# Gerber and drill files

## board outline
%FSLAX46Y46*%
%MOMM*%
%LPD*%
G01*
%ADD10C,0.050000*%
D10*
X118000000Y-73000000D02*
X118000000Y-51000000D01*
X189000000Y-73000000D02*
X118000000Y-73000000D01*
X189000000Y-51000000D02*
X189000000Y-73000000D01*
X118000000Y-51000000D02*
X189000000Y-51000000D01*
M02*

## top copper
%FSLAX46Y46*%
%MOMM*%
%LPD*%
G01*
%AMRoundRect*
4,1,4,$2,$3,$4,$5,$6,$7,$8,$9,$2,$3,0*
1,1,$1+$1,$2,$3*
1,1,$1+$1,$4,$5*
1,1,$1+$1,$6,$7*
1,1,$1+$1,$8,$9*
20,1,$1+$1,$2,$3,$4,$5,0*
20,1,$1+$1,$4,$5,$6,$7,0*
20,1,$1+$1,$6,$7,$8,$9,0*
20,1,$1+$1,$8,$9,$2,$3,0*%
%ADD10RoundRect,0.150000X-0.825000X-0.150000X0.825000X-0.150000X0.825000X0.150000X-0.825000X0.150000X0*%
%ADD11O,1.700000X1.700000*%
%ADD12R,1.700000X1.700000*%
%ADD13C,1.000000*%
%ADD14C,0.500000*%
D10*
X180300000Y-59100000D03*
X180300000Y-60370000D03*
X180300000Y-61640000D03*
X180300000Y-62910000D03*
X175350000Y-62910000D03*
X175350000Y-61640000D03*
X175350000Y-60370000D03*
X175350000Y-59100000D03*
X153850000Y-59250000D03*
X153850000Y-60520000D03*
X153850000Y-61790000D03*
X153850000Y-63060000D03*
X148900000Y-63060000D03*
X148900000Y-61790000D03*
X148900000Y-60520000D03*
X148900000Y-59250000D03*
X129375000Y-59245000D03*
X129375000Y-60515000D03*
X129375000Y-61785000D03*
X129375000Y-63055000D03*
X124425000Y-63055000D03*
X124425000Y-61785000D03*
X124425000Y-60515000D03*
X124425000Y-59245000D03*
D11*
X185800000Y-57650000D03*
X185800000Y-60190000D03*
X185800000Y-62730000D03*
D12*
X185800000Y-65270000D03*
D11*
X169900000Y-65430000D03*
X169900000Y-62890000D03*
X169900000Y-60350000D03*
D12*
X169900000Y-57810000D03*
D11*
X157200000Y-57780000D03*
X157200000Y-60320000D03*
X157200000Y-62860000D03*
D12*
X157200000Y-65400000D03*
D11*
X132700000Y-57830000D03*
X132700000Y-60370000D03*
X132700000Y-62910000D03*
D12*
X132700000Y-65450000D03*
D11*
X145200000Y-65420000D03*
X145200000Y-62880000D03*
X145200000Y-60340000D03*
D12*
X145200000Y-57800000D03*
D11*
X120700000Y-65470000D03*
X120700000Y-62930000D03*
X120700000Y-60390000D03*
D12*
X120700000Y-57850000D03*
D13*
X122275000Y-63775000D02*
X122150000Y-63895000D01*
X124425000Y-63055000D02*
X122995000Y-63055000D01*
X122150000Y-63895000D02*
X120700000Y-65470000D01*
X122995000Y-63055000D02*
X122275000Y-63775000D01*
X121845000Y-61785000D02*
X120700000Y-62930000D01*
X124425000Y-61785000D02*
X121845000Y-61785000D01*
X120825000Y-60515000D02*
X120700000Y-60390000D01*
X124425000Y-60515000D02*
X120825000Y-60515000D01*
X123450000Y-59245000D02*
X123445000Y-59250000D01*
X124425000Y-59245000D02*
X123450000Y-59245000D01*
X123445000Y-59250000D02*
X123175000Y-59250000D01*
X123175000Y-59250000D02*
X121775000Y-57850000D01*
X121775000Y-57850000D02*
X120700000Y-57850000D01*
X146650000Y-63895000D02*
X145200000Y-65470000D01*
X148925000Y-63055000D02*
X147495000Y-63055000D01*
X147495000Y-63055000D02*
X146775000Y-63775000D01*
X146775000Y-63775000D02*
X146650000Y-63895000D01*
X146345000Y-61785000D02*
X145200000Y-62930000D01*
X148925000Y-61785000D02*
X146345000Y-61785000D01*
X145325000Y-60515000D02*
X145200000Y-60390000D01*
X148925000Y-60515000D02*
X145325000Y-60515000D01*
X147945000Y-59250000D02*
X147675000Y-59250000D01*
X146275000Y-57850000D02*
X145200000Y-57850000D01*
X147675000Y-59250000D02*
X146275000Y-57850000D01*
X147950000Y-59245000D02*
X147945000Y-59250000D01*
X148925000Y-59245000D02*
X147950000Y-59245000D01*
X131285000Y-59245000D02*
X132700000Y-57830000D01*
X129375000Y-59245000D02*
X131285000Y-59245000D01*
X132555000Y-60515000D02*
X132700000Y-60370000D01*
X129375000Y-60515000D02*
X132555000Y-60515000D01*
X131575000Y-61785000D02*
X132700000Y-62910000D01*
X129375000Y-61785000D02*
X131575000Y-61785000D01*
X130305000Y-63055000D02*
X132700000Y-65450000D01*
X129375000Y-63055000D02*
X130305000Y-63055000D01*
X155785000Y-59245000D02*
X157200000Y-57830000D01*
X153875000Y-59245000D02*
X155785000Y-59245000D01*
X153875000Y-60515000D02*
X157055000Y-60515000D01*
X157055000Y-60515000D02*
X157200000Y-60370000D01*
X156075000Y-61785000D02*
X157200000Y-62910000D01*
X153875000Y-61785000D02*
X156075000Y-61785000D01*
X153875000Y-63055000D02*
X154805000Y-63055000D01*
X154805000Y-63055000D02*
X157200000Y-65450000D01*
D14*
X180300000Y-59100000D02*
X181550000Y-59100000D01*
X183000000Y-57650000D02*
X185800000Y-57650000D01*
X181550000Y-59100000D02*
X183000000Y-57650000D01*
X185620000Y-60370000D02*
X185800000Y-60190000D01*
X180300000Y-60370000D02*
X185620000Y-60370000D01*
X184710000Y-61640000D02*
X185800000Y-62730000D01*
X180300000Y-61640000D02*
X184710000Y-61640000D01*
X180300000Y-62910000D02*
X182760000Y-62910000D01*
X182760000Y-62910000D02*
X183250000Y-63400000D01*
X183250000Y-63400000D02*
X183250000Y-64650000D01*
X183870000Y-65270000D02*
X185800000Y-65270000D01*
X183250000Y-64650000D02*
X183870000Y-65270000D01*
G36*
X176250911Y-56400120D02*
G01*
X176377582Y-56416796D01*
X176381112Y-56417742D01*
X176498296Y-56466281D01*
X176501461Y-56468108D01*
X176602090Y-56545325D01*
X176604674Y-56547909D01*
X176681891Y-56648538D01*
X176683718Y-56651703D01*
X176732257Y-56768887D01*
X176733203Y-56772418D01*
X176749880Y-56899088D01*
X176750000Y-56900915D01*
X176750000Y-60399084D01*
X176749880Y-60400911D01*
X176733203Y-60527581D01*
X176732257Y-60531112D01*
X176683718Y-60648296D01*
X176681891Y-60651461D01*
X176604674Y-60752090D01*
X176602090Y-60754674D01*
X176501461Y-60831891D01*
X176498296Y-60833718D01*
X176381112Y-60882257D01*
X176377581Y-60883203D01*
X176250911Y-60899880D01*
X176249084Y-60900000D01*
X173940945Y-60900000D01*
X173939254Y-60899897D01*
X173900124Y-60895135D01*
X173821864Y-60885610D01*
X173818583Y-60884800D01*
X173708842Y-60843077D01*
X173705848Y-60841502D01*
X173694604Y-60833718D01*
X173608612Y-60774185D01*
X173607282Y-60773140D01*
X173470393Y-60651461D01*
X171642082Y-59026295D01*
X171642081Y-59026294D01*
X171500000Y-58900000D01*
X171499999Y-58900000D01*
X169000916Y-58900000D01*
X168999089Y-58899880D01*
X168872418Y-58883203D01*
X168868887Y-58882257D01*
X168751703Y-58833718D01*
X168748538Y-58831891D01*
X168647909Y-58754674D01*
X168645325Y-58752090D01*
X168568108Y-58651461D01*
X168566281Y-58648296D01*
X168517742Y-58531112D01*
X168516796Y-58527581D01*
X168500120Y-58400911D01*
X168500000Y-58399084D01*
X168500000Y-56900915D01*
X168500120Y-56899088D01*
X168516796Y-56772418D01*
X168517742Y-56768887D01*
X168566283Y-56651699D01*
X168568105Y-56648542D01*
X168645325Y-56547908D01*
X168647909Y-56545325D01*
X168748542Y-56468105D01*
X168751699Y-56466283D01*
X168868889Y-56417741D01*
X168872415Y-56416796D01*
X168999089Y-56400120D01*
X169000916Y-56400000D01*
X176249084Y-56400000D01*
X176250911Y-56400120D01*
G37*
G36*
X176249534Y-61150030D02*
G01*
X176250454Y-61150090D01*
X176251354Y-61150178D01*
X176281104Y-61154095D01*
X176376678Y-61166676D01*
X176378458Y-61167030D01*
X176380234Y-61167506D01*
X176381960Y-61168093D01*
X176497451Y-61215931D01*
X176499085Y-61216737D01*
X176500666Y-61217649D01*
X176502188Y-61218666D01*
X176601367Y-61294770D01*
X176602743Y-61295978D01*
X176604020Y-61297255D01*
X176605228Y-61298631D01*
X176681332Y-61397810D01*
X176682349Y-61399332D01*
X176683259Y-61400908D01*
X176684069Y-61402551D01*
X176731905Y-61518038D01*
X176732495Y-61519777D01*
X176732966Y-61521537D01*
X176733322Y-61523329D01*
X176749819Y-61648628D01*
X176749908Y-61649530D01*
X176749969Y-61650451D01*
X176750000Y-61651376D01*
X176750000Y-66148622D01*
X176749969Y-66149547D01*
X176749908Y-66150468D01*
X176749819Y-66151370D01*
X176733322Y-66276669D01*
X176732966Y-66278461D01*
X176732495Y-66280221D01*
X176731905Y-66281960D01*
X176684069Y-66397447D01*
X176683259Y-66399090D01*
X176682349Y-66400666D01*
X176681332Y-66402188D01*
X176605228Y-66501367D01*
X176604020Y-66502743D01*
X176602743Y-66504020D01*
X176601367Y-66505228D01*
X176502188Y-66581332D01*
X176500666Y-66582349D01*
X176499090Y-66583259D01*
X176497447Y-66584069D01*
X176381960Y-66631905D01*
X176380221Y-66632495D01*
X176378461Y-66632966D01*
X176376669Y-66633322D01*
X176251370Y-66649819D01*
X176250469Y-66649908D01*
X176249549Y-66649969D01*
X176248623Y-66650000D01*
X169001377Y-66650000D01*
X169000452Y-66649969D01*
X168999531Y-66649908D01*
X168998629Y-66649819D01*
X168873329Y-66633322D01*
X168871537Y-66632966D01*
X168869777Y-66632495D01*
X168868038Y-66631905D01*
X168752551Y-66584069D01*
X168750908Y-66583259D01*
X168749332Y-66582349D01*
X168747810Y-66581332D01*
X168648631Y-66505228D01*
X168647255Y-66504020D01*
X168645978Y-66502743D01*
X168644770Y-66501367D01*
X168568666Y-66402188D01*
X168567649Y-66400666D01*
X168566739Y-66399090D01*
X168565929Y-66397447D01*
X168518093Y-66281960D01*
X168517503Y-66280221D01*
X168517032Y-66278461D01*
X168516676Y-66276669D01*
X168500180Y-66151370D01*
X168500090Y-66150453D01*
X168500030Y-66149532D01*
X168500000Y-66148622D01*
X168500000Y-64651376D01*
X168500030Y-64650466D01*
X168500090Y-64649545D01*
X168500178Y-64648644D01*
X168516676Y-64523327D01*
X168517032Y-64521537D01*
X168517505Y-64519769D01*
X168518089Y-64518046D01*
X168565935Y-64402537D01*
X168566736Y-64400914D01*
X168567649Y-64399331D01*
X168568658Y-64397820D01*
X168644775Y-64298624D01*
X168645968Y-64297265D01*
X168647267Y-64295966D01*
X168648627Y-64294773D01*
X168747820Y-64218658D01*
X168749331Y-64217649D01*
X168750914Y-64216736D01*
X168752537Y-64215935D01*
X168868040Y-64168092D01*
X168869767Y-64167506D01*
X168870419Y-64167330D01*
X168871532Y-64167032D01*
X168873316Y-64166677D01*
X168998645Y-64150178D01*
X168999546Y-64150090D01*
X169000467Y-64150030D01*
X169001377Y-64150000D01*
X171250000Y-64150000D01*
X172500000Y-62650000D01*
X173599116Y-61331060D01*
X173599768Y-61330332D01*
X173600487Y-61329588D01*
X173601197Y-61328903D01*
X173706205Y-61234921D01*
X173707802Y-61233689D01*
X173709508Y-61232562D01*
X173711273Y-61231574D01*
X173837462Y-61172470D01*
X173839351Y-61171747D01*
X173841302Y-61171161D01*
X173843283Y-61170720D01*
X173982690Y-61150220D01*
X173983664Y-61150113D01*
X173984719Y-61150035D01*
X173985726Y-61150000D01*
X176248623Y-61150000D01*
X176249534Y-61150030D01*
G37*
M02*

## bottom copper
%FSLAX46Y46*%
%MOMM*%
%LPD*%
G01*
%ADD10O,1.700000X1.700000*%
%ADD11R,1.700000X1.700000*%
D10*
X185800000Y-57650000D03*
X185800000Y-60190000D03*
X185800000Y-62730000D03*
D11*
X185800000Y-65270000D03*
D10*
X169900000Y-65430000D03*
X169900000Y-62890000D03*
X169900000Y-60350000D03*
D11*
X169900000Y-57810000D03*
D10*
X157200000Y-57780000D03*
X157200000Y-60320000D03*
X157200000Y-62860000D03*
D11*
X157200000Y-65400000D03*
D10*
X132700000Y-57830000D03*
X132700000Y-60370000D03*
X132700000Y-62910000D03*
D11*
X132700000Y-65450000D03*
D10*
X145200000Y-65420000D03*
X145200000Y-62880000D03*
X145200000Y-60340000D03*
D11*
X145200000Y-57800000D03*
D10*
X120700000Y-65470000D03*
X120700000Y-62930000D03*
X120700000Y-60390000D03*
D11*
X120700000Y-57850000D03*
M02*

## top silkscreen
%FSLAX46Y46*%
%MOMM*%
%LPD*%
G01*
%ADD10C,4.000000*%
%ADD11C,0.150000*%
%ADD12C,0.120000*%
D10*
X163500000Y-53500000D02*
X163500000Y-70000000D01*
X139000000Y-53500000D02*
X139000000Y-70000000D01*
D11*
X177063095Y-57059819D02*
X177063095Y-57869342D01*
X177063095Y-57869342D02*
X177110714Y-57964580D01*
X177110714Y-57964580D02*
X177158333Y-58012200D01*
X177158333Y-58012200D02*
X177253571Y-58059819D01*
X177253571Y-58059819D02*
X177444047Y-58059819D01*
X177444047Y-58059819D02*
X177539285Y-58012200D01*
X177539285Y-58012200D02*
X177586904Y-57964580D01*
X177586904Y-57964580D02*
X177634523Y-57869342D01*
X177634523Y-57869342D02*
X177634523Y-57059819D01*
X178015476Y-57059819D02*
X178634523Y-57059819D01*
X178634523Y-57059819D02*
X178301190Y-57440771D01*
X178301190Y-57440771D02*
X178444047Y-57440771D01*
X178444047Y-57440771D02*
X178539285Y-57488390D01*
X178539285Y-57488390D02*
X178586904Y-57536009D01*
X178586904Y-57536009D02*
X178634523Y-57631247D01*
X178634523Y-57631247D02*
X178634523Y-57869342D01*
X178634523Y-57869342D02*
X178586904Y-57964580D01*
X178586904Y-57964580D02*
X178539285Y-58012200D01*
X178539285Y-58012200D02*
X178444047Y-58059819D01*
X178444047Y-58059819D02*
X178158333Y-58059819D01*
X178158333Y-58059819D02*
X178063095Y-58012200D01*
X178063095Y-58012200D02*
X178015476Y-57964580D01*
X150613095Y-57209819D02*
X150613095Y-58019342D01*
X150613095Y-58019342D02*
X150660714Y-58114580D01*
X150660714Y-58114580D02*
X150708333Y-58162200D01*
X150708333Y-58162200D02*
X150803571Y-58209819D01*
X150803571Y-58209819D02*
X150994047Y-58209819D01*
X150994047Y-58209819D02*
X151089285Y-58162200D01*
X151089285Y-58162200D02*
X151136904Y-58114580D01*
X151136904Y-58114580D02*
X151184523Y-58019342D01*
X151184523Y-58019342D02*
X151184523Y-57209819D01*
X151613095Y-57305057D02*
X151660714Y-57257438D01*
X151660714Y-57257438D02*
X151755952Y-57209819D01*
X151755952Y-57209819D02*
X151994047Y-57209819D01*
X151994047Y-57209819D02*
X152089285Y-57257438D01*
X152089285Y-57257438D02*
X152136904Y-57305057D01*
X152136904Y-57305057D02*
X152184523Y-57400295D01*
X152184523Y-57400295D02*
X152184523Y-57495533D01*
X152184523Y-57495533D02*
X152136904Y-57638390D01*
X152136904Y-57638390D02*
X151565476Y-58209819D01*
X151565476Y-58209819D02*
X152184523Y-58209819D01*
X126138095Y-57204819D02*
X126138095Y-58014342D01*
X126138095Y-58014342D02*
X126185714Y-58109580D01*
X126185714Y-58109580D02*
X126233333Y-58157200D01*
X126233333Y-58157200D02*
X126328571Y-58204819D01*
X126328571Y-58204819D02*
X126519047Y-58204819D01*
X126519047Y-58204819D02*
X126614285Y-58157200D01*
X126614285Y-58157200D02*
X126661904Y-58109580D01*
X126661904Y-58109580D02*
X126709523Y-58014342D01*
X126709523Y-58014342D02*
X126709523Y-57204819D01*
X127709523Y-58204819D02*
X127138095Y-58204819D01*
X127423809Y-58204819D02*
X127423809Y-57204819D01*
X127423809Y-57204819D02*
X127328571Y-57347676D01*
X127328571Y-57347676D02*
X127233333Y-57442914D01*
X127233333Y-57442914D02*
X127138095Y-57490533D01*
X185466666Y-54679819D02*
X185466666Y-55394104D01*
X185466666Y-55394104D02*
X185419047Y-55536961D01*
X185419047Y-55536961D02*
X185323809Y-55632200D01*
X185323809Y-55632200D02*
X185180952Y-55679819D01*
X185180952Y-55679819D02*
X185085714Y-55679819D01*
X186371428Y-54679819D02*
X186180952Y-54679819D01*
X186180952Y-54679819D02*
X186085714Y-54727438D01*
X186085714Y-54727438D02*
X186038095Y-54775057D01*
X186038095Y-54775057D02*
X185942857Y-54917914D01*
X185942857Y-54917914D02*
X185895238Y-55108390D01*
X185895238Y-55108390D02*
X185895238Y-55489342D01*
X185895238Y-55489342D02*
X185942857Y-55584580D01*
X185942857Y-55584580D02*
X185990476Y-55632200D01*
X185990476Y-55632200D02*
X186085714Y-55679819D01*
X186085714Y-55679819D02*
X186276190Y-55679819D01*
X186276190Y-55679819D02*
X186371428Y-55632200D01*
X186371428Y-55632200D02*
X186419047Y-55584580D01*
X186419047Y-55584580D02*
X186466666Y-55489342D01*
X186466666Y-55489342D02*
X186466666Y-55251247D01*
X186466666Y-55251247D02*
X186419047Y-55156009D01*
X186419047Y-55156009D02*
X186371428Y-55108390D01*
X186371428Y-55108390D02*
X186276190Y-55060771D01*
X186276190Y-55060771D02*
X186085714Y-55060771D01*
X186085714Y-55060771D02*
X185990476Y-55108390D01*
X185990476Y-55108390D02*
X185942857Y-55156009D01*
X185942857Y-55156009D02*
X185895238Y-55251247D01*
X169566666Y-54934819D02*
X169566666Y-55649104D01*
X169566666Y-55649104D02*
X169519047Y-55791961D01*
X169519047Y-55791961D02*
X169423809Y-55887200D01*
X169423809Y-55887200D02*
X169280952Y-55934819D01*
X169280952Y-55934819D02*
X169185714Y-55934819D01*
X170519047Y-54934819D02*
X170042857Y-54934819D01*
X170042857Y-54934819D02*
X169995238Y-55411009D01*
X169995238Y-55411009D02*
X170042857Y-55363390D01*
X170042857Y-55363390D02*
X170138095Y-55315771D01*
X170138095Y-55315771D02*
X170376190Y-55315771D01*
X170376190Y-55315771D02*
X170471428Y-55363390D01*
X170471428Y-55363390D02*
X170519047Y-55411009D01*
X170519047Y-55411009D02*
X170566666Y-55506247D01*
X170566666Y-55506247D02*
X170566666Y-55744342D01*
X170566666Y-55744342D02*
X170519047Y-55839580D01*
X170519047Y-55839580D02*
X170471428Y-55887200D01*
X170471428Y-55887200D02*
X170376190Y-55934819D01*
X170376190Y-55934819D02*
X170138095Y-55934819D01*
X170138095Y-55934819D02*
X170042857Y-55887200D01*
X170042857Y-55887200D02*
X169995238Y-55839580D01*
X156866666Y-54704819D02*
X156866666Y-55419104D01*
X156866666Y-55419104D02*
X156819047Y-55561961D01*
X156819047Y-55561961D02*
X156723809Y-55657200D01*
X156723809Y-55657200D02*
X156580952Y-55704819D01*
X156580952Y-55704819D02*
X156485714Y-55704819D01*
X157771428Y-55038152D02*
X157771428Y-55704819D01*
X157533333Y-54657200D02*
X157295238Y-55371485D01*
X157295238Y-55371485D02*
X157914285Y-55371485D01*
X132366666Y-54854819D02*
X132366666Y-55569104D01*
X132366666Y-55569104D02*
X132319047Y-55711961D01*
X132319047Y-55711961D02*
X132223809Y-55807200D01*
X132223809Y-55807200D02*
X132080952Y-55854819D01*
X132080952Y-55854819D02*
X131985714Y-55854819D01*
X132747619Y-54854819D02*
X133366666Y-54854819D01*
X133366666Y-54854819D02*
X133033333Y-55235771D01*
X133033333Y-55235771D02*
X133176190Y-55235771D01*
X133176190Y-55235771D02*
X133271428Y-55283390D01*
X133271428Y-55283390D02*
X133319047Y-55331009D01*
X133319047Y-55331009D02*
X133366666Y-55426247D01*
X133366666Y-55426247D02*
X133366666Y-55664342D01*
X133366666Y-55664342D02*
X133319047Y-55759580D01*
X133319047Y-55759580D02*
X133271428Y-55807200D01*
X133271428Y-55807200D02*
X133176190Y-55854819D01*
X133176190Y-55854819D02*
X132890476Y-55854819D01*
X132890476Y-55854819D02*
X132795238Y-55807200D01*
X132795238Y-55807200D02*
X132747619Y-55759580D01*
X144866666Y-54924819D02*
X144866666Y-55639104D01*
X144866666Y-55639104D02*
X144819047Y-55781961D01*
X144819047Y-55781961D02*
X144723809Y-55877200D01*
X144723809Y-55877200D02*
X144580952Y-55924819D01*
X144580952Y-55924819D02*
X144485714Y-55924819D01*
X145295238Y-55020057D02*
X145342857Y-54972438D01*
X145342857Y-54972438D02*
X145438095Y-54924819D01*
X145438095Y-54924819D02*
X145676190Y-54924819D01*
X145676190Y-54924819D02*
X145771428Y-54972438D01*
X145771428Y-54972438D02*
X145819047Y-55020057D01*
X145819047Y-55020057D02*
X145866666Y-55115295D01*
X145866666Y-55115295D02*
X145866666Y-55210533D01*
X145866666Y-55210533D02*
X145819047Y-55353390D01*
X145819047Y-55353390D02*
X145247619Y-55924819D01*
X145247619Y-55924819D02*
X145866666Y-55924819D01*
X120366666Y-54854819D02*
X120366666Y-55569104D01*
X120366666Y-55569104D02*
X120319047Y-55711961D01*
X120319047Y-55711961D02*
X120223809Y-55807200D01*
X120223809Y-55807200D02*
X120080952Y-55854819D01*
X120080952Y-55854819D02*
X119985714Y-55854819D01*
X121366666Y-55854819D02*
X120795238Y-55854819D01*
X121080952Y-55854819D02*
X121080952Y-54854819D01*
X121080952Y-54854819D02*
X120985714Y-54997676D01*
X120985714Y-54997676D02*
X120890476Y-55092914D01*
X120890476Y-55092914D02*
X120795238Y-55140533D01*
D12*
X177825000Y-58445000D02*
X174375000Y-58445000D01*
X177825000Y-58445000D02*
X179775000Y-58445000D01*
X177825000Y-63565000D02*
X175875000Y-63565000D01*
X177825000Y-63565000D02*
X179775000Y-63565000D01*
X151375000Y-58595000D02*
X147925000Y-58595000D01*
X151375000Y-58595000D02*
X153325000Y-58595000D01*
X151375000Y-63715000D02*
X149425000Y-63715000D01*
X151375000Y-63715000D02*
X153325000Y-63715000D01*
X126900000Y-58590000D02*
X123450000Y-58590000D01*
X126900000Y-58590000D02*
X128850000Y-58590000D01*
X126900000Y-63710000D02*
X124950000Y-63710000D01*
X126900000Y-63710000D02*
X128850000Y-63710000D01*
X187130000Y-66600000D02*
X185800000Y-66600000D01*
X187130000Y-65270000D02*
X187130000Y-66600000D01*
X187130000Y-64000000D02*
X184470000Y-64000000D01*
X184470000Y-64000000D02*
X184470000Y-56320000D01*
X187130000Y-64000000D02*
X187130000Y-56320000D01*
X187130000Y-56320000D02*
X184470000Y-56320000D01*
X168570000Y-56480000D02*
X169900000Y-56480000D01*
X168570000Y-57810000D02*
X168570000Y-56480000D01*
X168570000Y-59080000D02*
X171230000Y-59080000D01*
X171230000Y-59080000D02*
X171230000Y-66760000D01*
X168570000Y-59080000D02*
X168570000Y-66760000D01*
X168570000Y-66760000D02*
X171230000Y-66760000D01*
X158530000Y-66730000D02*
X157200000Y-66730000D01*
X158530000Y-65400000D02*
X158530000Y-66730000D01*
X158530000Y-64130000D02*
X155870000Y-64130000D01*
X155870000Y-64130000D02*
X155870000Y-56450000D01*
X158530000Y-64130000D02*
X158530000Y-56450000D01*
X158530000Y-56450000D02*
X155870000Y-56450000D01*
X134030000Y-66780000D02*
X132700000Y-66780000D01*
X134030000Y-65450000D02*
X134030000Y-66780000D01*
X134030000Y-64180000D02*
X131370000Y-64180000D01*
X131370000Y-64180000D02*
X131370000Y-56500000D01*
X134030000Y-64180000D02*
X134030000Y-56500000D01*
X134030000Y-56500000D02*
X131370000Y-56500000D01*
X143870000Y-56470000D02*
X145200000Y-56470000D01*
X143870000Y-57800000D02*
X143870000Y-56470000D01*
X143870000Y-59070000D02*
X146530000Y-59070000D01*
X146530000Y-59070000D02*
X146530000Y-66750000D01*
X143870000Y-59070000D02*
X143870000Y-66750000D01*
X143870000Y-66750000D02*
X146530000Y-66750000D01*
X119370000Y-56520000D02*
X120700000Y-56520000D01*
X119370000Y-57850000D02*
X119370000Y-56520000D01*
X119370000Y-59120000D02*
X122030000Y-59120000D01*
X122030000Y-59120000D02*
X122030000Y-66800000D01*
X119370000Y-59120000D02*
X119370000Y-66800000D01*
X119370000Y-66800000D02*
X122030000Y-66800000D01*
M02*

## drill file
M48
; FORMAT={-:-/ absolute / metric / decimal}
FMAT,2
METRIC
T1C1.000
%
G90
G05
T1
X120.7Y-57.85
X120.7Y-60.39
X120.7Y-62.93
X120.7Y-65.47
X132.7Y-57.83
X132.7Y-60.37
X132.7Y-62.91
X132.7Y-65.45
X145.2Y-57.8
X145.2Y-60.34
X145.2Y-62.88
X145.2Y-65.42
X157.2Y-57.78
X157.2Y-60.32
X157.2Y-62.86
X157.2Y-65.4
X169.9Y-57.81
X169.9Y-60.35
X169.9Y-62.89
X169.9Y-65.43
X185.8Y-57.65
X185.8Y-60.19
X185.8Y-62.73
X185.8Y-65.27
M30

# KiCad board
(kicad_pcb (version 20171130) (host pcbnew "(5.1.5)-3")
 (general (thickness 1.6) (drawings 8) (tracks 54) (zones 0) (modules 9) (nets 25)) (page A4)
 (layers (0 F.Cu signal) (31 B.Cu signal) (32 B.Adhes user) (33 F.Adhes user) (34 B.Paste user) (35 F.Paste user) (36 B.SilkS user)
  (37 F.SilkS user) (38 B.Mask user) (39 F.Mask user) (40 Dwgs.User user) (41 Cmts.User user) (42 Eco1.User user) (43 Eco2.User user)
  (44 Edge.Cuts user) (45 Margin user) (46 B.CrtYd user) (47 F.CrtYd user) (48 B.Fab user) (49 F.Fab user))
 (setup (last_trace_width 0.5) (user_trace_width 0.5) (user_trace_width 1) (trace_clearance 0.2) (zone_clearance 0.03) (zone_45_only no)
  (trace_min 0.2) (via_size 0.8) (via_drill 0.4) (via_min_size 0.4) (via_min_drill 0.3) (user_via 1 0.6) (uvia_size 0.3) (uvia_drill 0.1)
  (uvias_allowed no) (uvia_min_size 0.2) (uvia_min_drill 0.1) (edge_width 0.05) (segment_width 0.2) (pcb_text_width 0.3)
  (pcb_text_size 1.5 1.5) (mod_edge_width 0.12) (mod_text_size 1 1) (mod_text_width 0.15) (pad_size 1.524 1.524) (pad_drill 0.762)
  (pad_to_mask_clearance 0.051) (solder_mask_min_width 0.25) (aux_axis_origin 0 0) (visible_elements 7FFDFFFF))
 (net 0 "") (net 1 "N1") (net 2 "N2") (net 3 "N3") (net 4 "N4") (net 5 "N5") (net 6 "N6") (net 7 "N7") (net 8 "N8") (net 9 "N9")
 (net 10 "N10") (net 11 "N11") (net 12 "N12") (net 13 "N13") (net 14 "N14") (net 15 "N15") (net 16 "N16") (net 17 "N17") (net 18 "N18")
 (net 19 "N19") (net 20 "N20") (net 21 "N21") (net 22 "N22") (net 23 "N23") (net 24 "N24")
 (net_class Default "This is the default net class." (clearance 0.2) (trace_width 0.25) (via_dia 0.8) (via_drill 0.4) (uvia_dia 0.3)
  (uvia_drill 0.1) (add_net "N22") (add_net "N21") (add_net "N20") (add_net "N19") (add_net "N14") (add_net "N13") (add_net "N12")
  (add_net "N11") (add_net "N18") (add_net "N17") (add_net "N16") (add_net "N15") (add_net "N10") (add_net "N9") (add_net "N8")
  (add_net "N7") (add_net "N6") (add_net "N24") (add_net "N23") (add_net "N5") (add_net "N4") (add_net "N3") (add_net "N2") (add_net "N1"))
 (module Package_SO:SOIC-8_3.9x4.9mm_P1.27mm (layer F.Cu) (at 177.825 61.005)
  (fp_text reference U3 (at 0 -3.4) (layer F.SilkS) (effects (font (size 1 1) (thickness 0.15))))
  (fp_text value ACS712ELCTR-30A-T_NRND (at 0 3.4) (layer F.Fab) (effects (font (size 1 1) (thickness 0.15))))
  (fp_line (start 0 -2.56) (end -3.45 -2.56) (layer F.SilkS) (width 0.12))
  (fp_line (start 0 -2.56) (end 1.95 -2.56) (layer F.SilkS) (width 0.12))
  (fp_line (start 0 2.56) (end -1.95 2.56) (layer F.SilkS) (width 0.12))
  (fp_line (start 0 2.56) (end 1.95 2.56) (layer F.SilkS) (width 0.12))
  (pad 8 smd roundrect (at 2.475 -1.905) (size 1.95 0.6) (layers F.Cu F.Paste F.Mask) (roundrect_rratio 0.25) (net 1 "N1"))
  (pad 7 smd roundrect (at 2.475 -0.635) (size 1.95 0.6) (layers F.Cu F.Paste F.Mask) (roundrect_rratio 0.25) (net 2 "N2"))
  (pad 6 smd roundrect (at 2.475 0.635) (size 1.95 0.6) (layers F.Cu F.Paste F.Mask) (roundrect_rratio 0.25) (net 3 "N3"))
  (pad 5 smd roundrect (at 2.475 1.905) (size 1.95 0.6) (layers F.Cu F.Paste F.Mask) (roundrect_rratio 0.25) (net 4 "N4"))
  (pad 4 smd roundrect (at -2.475 1.905) (size 1.95 0.6) (layers F.Cu F.Paste F.Mask) (roundrect_rratio 0.25) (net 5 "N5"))
  (pad 3 smd roundrect (at -2.475 0.635) (size 1.95 0.6) (layers F.Cu F.Paste F.Mask) (roundrect_rratio 0.25) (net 5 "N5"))
  (pad 2 smd roundrect (at -2.475 -0.635) (size 1.95 0.6) (layers F.Cu F.Paste F.Mask) (roundrect_rratio 0.25) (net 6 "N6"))
  (pad 1 smd roundrect (at -2.475 -1.905) (size 1.95 0.6) (layers F.Cu F.Paste F.Mask) (roundrect_rratio 0.25) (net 6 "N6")))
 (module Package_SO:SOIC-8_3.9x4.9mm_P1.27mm (layer F.Cu) (at 151.375 61.155)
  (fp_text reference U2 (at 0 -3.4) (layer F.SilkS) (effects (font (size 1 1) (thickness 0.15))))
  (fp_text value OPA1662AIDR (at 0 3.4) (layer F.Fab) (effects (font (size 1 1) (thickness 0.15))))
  (fp_line (start 0 -2.56) (end -3.45 -2.56) (layer F.SilkS) (width 0.12))
  (fp_line (start 0 -2.56) (end 1.95 -2.56) (layer F.SilkS) (width 0.12))
  (fp_line (start 0 2.56) (end -1.95 2.56) (layer F.SilkS) (width 0.12))
  (fp_line (start 0 2.56) (end 1.95 2.56) (layer F.SilkS) (width 0.12))
  (pad 8 smd roundrect (at 2.475 -1.905) (size 1.95 0.6) (layers F.Cu F.Paste F.Mask) (roundrect_rratio 0.25) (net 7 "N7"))
  (pad 7 smd roundrect (at 2.475 -0.635) (size 1.95 0.6) (layers F.Cu F.Paste F.Mask) (roundrect_rratio 0.25) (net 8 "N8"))
  (pad 6 smd roundrect (at 2.475 0.635) (size 1.95 0.6) (layers F.Cu F.Paste F.Mask) (roundrect_rratio 0.25) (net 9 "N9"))
  (pad 5 smd roundrect (at 2.475 1.905) (size 1.95 0.6) (layers F.Cu F.Paste F.Mask) (roundrect_rratio 0.25) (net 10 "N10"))
  (pad 4 smd roundrect (at -2.475 1.905) (size 1.95 0.6) (layers F.Cu F.Paste F.Mask) (roundrect_rratio 0.25) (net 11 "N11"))
  (pad 3 smd roundrect (at -2.475 0.635) (size 1.95 0.6) (layers F.Cu F.Paste F.Mask) (roundrect_rratio 0.25) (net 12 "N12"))
  (pad 2 smd roundrect (at -2.475 -0.635) (size 1.95 0.6) (layers F.Cu F.Paste F.Mask) (roundrect_rratio 0.25) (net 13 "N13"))
  (pad 1 smd roundrect (at -2.475 -1.905) (size 1.95 0.6) (layers F.Cu F.Paste F.Mask) (roundrect_rratio 0.25) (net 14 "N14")))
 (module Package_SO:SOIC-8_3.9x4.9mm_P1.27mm (layer F.Cu) (at 126.9 61.15)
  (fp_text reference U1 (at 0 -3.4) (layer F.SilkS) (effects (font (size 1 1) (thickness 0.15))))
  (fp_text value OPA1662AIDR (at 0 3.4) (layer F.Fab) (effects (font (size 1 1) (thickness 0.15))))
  (fp_line (start 0 -2.56) (end -3.45 -2.56) (layer F.SilkS) (width 0.12))
  (fp_line (start 0 -2.56) (end 1.95 -2.56) (layer F.SilkS) (width 0.12))
  (fp_line (start 0 2.56) (end -1.95 2.56) (layer F.SilkS) (width 0.12))
  (fp_line (start 0 2.56) (end 1.95 2.56) (layer F.SilkS) (width 0.12))
  (pad 8 smd roundrect (at 2.475 -1.905) (size 1.95 0.6) (layers F.Cu F.Paste F.Mask) (roundrect_rratio 0.25) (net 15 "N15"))
  (pad 7 smd roundrect (at 2.475 -0.635) (size 1.95 0.6) (layers F.Cu F.Paste F.Mask) (roundrect_rratio 0.25) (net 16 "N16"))
  (pad 6 smd roundrect (at 2.475 0.635) (size 1.95 0.6) (layers F.Cu F.Paste F.Mask) (roundrect_rratio 0.25) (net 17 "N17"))
  (pad 5 smd roundrect (at 2.475 1.905) (size 1.95 0.6) (layers F.Cu F.Paste F.Mask) (roundrect_rratio 0.25) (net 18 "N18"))
  (pad 4 smd roundrect (at -2.475 1.905) (size 1.95 0.6) (layers F.Cu F.Paste F.Mask) (roundrect_rratio 0.25) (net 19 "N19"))
  (pad 3 smd roundrect (at -2.475 0.635) (size 1.95 0.6) (layers F.Cu F.Paste F.Mask) (roundrect_rratio 0.25) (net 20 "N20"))
  (pad 2 smd roundrect (at -2.475 -0.635) (size 1.95 0.6) (layers F.Cu F.Paste F.Mask) (roundrect_rratio 0.25) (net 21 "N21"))
  (pad 1 smd roundrect (at -2.475 -1.905) (size 1.95 0.6) (layers F.Cu F.Paste F.Mask) (roundrect_rratio 0.25) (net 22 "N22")))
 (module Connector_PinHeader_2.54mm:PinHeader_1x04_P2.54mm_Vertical (layer F.Cu) (at 185.8 65.27 180)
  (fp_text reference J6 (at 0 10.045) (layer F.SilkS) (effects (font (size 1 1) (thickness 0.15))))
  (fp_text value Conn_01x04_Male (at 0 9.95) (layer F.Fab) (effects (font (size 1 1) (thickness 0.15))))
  (fp_line (start -1.33 -1.33) (end 0 -1.33) (layer F.SilkS) (width 0.12))
  (fp_line (start -1.33 0) (end -1.33 -1.33) (layer F.SilkS) (width 0.12))
  (fp_line (start -1.33 1.27) (end 1.33 1.27) (layer F.SilkS) (width 0.12))
  (fp_line (start 1.33 1.27) (end 1.33 8.95) (layer F.SilkS) (width 0.12))
  (fp_line (start -1.33 1.27) (end -1.33 8.95) (layer F.SilkS) (width 0.12))
  (fp_line (start -1.33 8.95) (end 1.33 8.95) (layer F.SilkS) (width 0.12))
  (pad 4 thru_hole oval (at 0 7.62 180) (size 1.7 1.7) (drill 1) (layers *.Cu *.Mask) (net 1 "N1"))
  (pad 3 thru_hole oval (at 0 5.08 180) (size 1.7 1.7) (drill 1) (layers *.Cu *.Mask) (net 2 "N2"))
  (pad 2 thru_hole oval (at 0 2.54 180) (size 1.7 1.7) (drill 1) (layers *.Cu *.Mask) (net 3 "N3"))
  (pad 1 thru_hole rect (at 0 0 180) (size 1.7 1.7) (drill 1) (layers *.Cu *.Mask) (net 4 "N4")))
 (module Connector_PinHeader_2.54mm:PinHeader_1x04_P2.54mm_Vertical (layer F.Cu) (at 169.9 57.81)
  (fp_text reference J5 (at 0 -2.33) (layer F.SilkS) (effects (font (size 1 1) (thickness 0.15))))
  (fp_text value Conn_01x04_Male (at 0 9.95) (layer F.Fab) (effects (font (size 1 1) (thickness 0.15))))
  (fp_line (start -1.33 -1.33) (end 0 -1.33) (layer F.SilkS) (width 0.12))
  (fp_line (start -1.33 0) (end -1.33 -1.33) (layer F.SilkS) (width 0.12))
  (fp_line (start -1.33 1.27) (end 1.33 1.27) (layer F.SilkS) (width 0.12))
  (fp_line (start 1.33 1.27) (end 1.33 8.95) (layer F.SilkS) (width 0.12))
  (fp_line (start -1.33 1.27) (end -1.33 8.95) (layer F.SilkS) (width 0.12))
  (fp_line (start -1.33 8.95) (end 1.33 8.95) (layer F.SilkS) (width 0.12))
  (pad 4 thru_hole oval (at 0 7.62) (size 1.7 1.7) (drill 1) (layers *.Cu *.Mask) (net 5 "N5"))
  (pad 3 thru_hole oval (at 0 5.08) (size 1.7 1.7) (drill 1) (layers *.Cu *.Mask) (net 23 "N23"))
  (pad 2 thru_hole oval (at 0 2.54) (size 1.7 1.7) (drill 1) (layers *.Cu *.Mask) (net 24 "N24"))
  (pad 1 thru_hole rect (at 0 0) (size 1.7 1.7) (drill 1) (layers *.Cu *.Mask) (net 6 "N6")))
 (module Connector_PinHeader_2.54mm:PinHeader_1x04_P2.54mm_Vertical (layer F.Cu) (at 157.2 65.4 180)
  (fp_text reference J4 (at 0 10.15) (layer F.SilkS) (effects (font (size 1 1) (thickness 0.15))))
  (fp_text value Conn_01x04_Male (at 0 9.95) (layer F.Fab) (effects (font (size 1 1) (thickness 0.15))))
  (fp_line (start -1.33 -1.33) (end 0 -1.33) (layer F.SilkS) (width 0.12))
  (fp_line (start -1.33 0) (end -1.33 -1.33) (layer F.SilkS) (width 0.12))
  (fp_line (start -1.33 1.27) (end 1.33 1.27) (layer F.SilkS) (width 0.12))
  (fp_line (start 1.33 1.27) (end 1.33 8.95) (layer F.SilkS) (width 0.12))
  (fp_line (start -1.33 1.27) (end -1.33 8.95) (layer F.SilkS) (width 0.12))
  (fp_line (start -1.33 8.95) (end 1.33 8.95) (layer F.SilkS) (width 0.12))
  (pad 4 thru_hole oval (at 0 7.62 180) (size 1.7 1.7) (drill 1) (layers *.Cu *.Mask) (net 7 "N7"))
  (pad 3 thru_hole oval (at 0 5.08 180) (size 1.7 1.7) (drill 1) (layers *.Cu *.Mask) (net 8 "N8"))
  (pad 2 thru_hole oval (at 0 2.54 180) (size 1.7 1.7) (drill 1) (layers *.Cu *.Mask) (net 9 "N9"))
  (pad 1 thru_hole rect (at 0 0 180) (size 1.7 1.7) (drill 1) (layers *.Cu *.Mask) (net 10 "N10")))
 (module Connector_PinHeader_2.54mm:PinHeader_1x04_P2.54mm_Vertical (layer F.Cu) (at 132.7 65.45 180)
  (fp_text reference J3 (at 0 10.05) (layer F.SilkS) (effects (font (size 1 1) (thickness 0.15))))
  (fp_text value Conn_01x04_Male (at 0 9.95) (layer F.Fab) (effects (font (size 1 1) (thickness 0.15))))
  (fp_line (start -1.33 -1.33) (end 0 -1.33) (layer F.SilkS) (width 0.12))
  (fp_line (start -1.33 0) (end -1.33 -1.33) (layer F.SilkS) (width 0.12))
  (fp_line (start -1.33 1.27) (end 1.33 1.27) (layer F.SilkS) (width 0.12))
  (fp_line (start 1.33 1.27) (end 1.33 8.95) (layer F.SilkS) (width 0.12))
  (fp_line (start -1.33 1.27) (end -1.33 8.95) (layer F.SilkS) (width 0.12))
  (fp_line (start -1.33 8.95) (end 1.33 8.95) (layer F.SilkS) (width 0.12))
  (pad 4 thru_hole oval (at 0 7.62 180) (size 1.7 1.7) (drill 1) (layers *.Cu *.Mask) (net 15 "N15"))
  (pad 3 thru_hole oval (at 0 5.08 180) (size 1.7 1.7) (drill 1) (layers *.Cu *.Mask) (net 16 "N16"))
  (pad 2 thru_hole oval (at 0 2.54 180) (size 1.7 1.7) (drill 1) (layers *.Cu *.Mask) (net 17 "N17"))
  (pad 1 thru_hole rect (at 0 0 180) (size 1.7 1.7) (drill 1) (layers *.Cu *.Mask) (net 18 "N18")))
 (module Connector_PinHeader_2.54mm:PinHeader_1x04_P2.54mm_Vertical (layer F.Cu) (at 145.2 57.8)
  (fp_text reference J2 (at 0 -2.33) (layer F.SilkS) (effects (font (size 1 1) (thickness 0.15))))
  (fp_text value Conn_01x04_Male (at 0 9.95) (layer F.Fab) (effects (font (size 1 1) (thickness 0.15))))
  (fp_line (start -1.33 -1.33) (end 0 -1.33) (layer F.SilkS) (width 0.12))
  (fp_line (start -1.33 0) (end -1.33 -1.33) (layer F.SilkS) (width 0.12))
  (fp_line (start -1.33 1.27) (end 1.33 1.27) (layer F.SilkS) (width 0.12))
  (fp_line (start 1.33 1.27) (end 1.33 8.95) (layer F.SilkS) (width 0.12))
  (fp_line (start -1.33 1.27) (end -1.33 8.95) (layer F.SilkS) (width 0.12))
  (fp_line (start -1.33 8.95) (end 1.33 8.95) (layer F.SilkS) (width 0.12))
  (pad 4 thru_hole oval (at 0 7.62) (size 1.7 1.7) (drill 1) (layers *.Cu *.Mask) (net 11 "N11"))
  (pad 3 thru_hole oval (at 0 5.08) (size 1.7 1.7) (drill 1) (layers *.Cu *.Mask) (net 12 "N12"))
  (pad 2 thru_hole oval (at 0 2.54) (size 1.7 1.7) (drill 1) (layers *.Cu *.Mask) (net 13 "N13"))
  (pad 1 thru_hole rect (at 0 0) (size 1.7 1.7) (drill 1) (layers *.Cu *.Mask) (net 14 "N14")))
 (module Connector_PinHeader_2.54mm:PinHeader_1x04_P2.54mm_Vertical (layer F.Cu) (at 120.7 57.85)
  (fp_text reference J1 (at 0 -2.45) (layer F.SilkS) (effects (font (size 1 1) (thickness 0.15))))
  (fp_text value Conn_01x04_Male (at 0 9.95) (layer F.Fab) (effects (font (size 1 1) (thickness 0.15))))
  (fp_line (start -1.33 -1.33) (end 0 -1.33) (layer F.SilkS) (width 0.12))
  (fp_line (start -1.33 0) (end -1.33 -1.33) (layer F.SilkS) (width 0.12))
  (fp_line (start -1.33 1.27) (end 1.33 1.27) (layer F.SilkS) (width 0.12))
  (fp_line (start 1.33 1.27) (end 1.33 8.95) (layer F.SilkS) (width 0.12))
  (fp_line (start -1.33 1.27) (end -1.33 8.95) (layer F.SilkS) (width 0.12))
  (fp_line (start -1.33 8.95) (end 1.33 8.95) (layer F.SilkS) (width 0.12))
  (pad 4 thru_hole oval (at 0 7.62) (size 1.7 1.7) (drill 1) (layers *.Cu *.Mask) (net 19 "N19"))
  (pad 3 thru_hole oval (at 0 5.08) (size 1.7 1.7) (drill 1) (layers *.Cu *.Mask) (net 20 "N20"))
  (pad 2 thru_hole oval (at 0 2.54) (size 1.7 1.7) (drill 1) (layers *.Cu *.Mask) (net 21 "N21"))
  (pad 1 thru_hole rect (at 0 0) (size 1.7 1.7) (drill 1) (layers *.Cu *.Mask) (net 22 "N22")))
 (gr_line (start 118 73) (end 118 51) (layer Edge.Cuts) (width 0.05))
 (gr_line (start 189 73) (end 118 73) (layer Edge.Cuts) (width 0.05))
 (gr_line (start 189 51) (end 189 73) (layer Edge.Cuts) (width 0.05))
 (gr_line (start 118 51) (end 189 51) (layer Edge.Cuts) (width 0.05))
 (gr_line (start 163.5 53.5) (end 163.5 70) (layer F.SilkS) (width 4))
 (gr_line (start 139 53.5) (end 139 70) (layer F.SilkS) (width 4))
 (segment (start 122.275 63.775) (end 122.15 63.895) (width 1) (layer F.Cu) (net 19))
 (segment (start 124.425 63.055) (end 122.995 63.055) (width 1) (layer F.Cu) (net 19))
 (segment (start 122.15 63.895) (end 120.7 65.47) (width 1) (layer F.Cu) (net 19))
 (segment (start 122.995 63.055) (end 122.275 63.775) (width 1) (layer F.Cu) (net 19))
 (segment (start 121.845 61.785) (end 120.7 62.93) (width 1) (layer F.Cu) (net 20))
 (segment (start 124.425 61.785) (end 121.845 61.785) (width 1) (layer F.Cu) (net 20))
 (segment (start 120.825 60.515) (end 120.7 60.39) (width 1) (layer F.Cu) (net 21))
 (segment (start 124.425 60.515) (end 120.825 60.515) (width 1) (layer F.Cu) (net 21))
 (segment (start 123.45 59.245) (end 123.445 59.25) (width 1) (layer F.Cu) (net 22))
 (segment (start 124.425 59.245) (end 123.45 59.245) (width 1) (layer F.Cu) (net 22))
 (segment (start 123.445 59.25) (end 123.175 59.25) (width 1) (layer F.Cu) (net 22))
 (segment (start 123.175 59.25) (end 121.775 57.85) (width 1) (layer F.Cu) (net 22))
 (segment (start 121.775 57.85) (end 120.7 57.85) (width 1) (layer F.Cu) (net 22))
 (segment (start 146.65 63.895) (end 145.2 65.47) (width 1) (layer F.Cu) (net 11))
 (segment (start 148.925 63.055) (end 147.495 63.055) (width 1) (layer F.Cu) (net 11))
 (segment (start 147.495 63.055) (end 146.775 63.775) (width 1) (layer F.Cu) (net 11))
 (segment (start 146.775 63.775) (end 146.65 63.895) (width 1) (layer F.Cu) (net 11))
 (segment (start 146.345 61.785) (end 145.2 62.93) (width 1) (layer F.Cu) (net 12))
 (segment (start 148.925 61.785) (end 146.345 61.785) (width 1) (layer F.Cu) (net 12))
 (segment (start 145.325 60.515) (end 145.2 60.39) (width 1) (layer F.Cu) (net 13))
 (segment (start 148.925 60.515) (end 145.325 60.515) (width 1) (layer F.Cu) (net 13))
 (segment (start 147.945 59.25) (end 147.675 59.25) (width 1) (layer F.Cu) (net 14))
 (segment (start 146.275 57.85) (end 145.2 57.85) (width 1) (layer F.Cu) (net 14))
 (segment (start 147.675 59.25) (end 146.275 57.85) (width 1) (layer F.Cu) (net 14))
 (segment (start 147.95 59.245) (end 147.945 59.25) (width 1) (layer F.Cu) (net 14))
 (segment (start 148.925 59.245) (end 147.95 59.245) (width 1) (layer F.Cu) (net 14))
 (segment (start 131.285 59.245) (end 132.7 57.83) (width 1) (layer F.Cu) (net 15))
 (segment (start 129.375 59.245) (end 131.285 59.245) (width 1) (layer F.Cu) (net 15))
 (segment (start 132.555 60.515) (end 132.7 60.37) (width 1) (layer F.Cu) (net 16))
 (segment (start 129.375 60.515) (end 132.555 60.515) (width 1) (layer F.Cu) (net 16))
 (segment (start 131.575 61.785) (end 132.7 62.91) (width 1) (layer F.Cu) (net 17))
 (segment (start 129.375 61.785) (end 131.575 61.785) (width 1) (layer F.Cu) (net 17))
 (segment (start 130.305 63.055) (end 132.7 65.45) (width 1) (layer F.Cu) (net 18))
 (segment (start 129.375 63.055) (end 130.305 63.055) (width 1) (layer F.Cu) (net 18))
 (segment (start 155.785 59.245) (end 157.2 57.83) (width 1) (layer F.Cu) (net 7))
 (segment (start 153.875 59.245) (end 155.785 59.245) (width 1) (layer F.Cu) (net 7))
 (segment (start 153.875 60.515) (end 157.055 60.515) (width 1) (layer F.Cu) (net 8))
 (segment (start 157.055 60.515) (end 157.2 60.37) (width 1) (layer F.Cu) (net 8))
 (segment (start 156.075 61.785) (end 157.2 62.91) (width 1) (layer F.Cu) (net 9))
 (segment (start 153.875 61.785) (end 156.075 61.785) (width 1) (layer F.Cu) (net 9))
 (segment (start 153.875 63.055) (end 154.805 63.055) (width 1) (layer F.Cu) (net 10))
 (segment (start 154.805 63.055) (end 157.2 65.45) (width 1) (layer F.Cu) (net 10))
 (segment (start 180.3 59.1) (end 181.55 59.1) (width 0.5) (layer F.Cu) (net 1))
 (segment (start 183 57.65) (end 185.8 57.65) (width 0.5) (layer F.Cu) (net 1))
 (segment (start 181.55 59.1) (end 183 57.65) (width 0.5) (layer F.Cu) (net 1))
 (segment (start 185.62 60.37) (end 185.8 60.19) (width 0.5) (layer F.Cu) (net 2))
 (segment (start 180.3 60.37) (end 185.62 60.37) (width 0.5) (layer F.Cu) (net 2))
 (segment (start 184.71 61.64) (end 185.8 62.73) (width 0.5) (layer F.Cu) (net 3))
 (segment (start 180.3 61.64) (end 184.71 61.64) (width 0.5) (layer F.Cu) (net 3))
 (segment (start 180.3 62.91) (end 182.76 62.91) (width 0.5) (layer F.Cu) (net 4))
 (segment (start 182.76 62.91) (end 183.25 63.4) (width 0.5) (layer F.Cu) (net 4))
 (segment (start 183.25 63.4) (end 183.25 64.65) (width 0.5) (layer F.Cu) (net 4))
 (segment (start 183.87 65.27) (end 185.8 65.27) (width 0.5) (layer F.Cu) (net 4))
 (segment (start 183.25 64.65) (end 183.87 65.27) (width 0.5) (layer F.Cu) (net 4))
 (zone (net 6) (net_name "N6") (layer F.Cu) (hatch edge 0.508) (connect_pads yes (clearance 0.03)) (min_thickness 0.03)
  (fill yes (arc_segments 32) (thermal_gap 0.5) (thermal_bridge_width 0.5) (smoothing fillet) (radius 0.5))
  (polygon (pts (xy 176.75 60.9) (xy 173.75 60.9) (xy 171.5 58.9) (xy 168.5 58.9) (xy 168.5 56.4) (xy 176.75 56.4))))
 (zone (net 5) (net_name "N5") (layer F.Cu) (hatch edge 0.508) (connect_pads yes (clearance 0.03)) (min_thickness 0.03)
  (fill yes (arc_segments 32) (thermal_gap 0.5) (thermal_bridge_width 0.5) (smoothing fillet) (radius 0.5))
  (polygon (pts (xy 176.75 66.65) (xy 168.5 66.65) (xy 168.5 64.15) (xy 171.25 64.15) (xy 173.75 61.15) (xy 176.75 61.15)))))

